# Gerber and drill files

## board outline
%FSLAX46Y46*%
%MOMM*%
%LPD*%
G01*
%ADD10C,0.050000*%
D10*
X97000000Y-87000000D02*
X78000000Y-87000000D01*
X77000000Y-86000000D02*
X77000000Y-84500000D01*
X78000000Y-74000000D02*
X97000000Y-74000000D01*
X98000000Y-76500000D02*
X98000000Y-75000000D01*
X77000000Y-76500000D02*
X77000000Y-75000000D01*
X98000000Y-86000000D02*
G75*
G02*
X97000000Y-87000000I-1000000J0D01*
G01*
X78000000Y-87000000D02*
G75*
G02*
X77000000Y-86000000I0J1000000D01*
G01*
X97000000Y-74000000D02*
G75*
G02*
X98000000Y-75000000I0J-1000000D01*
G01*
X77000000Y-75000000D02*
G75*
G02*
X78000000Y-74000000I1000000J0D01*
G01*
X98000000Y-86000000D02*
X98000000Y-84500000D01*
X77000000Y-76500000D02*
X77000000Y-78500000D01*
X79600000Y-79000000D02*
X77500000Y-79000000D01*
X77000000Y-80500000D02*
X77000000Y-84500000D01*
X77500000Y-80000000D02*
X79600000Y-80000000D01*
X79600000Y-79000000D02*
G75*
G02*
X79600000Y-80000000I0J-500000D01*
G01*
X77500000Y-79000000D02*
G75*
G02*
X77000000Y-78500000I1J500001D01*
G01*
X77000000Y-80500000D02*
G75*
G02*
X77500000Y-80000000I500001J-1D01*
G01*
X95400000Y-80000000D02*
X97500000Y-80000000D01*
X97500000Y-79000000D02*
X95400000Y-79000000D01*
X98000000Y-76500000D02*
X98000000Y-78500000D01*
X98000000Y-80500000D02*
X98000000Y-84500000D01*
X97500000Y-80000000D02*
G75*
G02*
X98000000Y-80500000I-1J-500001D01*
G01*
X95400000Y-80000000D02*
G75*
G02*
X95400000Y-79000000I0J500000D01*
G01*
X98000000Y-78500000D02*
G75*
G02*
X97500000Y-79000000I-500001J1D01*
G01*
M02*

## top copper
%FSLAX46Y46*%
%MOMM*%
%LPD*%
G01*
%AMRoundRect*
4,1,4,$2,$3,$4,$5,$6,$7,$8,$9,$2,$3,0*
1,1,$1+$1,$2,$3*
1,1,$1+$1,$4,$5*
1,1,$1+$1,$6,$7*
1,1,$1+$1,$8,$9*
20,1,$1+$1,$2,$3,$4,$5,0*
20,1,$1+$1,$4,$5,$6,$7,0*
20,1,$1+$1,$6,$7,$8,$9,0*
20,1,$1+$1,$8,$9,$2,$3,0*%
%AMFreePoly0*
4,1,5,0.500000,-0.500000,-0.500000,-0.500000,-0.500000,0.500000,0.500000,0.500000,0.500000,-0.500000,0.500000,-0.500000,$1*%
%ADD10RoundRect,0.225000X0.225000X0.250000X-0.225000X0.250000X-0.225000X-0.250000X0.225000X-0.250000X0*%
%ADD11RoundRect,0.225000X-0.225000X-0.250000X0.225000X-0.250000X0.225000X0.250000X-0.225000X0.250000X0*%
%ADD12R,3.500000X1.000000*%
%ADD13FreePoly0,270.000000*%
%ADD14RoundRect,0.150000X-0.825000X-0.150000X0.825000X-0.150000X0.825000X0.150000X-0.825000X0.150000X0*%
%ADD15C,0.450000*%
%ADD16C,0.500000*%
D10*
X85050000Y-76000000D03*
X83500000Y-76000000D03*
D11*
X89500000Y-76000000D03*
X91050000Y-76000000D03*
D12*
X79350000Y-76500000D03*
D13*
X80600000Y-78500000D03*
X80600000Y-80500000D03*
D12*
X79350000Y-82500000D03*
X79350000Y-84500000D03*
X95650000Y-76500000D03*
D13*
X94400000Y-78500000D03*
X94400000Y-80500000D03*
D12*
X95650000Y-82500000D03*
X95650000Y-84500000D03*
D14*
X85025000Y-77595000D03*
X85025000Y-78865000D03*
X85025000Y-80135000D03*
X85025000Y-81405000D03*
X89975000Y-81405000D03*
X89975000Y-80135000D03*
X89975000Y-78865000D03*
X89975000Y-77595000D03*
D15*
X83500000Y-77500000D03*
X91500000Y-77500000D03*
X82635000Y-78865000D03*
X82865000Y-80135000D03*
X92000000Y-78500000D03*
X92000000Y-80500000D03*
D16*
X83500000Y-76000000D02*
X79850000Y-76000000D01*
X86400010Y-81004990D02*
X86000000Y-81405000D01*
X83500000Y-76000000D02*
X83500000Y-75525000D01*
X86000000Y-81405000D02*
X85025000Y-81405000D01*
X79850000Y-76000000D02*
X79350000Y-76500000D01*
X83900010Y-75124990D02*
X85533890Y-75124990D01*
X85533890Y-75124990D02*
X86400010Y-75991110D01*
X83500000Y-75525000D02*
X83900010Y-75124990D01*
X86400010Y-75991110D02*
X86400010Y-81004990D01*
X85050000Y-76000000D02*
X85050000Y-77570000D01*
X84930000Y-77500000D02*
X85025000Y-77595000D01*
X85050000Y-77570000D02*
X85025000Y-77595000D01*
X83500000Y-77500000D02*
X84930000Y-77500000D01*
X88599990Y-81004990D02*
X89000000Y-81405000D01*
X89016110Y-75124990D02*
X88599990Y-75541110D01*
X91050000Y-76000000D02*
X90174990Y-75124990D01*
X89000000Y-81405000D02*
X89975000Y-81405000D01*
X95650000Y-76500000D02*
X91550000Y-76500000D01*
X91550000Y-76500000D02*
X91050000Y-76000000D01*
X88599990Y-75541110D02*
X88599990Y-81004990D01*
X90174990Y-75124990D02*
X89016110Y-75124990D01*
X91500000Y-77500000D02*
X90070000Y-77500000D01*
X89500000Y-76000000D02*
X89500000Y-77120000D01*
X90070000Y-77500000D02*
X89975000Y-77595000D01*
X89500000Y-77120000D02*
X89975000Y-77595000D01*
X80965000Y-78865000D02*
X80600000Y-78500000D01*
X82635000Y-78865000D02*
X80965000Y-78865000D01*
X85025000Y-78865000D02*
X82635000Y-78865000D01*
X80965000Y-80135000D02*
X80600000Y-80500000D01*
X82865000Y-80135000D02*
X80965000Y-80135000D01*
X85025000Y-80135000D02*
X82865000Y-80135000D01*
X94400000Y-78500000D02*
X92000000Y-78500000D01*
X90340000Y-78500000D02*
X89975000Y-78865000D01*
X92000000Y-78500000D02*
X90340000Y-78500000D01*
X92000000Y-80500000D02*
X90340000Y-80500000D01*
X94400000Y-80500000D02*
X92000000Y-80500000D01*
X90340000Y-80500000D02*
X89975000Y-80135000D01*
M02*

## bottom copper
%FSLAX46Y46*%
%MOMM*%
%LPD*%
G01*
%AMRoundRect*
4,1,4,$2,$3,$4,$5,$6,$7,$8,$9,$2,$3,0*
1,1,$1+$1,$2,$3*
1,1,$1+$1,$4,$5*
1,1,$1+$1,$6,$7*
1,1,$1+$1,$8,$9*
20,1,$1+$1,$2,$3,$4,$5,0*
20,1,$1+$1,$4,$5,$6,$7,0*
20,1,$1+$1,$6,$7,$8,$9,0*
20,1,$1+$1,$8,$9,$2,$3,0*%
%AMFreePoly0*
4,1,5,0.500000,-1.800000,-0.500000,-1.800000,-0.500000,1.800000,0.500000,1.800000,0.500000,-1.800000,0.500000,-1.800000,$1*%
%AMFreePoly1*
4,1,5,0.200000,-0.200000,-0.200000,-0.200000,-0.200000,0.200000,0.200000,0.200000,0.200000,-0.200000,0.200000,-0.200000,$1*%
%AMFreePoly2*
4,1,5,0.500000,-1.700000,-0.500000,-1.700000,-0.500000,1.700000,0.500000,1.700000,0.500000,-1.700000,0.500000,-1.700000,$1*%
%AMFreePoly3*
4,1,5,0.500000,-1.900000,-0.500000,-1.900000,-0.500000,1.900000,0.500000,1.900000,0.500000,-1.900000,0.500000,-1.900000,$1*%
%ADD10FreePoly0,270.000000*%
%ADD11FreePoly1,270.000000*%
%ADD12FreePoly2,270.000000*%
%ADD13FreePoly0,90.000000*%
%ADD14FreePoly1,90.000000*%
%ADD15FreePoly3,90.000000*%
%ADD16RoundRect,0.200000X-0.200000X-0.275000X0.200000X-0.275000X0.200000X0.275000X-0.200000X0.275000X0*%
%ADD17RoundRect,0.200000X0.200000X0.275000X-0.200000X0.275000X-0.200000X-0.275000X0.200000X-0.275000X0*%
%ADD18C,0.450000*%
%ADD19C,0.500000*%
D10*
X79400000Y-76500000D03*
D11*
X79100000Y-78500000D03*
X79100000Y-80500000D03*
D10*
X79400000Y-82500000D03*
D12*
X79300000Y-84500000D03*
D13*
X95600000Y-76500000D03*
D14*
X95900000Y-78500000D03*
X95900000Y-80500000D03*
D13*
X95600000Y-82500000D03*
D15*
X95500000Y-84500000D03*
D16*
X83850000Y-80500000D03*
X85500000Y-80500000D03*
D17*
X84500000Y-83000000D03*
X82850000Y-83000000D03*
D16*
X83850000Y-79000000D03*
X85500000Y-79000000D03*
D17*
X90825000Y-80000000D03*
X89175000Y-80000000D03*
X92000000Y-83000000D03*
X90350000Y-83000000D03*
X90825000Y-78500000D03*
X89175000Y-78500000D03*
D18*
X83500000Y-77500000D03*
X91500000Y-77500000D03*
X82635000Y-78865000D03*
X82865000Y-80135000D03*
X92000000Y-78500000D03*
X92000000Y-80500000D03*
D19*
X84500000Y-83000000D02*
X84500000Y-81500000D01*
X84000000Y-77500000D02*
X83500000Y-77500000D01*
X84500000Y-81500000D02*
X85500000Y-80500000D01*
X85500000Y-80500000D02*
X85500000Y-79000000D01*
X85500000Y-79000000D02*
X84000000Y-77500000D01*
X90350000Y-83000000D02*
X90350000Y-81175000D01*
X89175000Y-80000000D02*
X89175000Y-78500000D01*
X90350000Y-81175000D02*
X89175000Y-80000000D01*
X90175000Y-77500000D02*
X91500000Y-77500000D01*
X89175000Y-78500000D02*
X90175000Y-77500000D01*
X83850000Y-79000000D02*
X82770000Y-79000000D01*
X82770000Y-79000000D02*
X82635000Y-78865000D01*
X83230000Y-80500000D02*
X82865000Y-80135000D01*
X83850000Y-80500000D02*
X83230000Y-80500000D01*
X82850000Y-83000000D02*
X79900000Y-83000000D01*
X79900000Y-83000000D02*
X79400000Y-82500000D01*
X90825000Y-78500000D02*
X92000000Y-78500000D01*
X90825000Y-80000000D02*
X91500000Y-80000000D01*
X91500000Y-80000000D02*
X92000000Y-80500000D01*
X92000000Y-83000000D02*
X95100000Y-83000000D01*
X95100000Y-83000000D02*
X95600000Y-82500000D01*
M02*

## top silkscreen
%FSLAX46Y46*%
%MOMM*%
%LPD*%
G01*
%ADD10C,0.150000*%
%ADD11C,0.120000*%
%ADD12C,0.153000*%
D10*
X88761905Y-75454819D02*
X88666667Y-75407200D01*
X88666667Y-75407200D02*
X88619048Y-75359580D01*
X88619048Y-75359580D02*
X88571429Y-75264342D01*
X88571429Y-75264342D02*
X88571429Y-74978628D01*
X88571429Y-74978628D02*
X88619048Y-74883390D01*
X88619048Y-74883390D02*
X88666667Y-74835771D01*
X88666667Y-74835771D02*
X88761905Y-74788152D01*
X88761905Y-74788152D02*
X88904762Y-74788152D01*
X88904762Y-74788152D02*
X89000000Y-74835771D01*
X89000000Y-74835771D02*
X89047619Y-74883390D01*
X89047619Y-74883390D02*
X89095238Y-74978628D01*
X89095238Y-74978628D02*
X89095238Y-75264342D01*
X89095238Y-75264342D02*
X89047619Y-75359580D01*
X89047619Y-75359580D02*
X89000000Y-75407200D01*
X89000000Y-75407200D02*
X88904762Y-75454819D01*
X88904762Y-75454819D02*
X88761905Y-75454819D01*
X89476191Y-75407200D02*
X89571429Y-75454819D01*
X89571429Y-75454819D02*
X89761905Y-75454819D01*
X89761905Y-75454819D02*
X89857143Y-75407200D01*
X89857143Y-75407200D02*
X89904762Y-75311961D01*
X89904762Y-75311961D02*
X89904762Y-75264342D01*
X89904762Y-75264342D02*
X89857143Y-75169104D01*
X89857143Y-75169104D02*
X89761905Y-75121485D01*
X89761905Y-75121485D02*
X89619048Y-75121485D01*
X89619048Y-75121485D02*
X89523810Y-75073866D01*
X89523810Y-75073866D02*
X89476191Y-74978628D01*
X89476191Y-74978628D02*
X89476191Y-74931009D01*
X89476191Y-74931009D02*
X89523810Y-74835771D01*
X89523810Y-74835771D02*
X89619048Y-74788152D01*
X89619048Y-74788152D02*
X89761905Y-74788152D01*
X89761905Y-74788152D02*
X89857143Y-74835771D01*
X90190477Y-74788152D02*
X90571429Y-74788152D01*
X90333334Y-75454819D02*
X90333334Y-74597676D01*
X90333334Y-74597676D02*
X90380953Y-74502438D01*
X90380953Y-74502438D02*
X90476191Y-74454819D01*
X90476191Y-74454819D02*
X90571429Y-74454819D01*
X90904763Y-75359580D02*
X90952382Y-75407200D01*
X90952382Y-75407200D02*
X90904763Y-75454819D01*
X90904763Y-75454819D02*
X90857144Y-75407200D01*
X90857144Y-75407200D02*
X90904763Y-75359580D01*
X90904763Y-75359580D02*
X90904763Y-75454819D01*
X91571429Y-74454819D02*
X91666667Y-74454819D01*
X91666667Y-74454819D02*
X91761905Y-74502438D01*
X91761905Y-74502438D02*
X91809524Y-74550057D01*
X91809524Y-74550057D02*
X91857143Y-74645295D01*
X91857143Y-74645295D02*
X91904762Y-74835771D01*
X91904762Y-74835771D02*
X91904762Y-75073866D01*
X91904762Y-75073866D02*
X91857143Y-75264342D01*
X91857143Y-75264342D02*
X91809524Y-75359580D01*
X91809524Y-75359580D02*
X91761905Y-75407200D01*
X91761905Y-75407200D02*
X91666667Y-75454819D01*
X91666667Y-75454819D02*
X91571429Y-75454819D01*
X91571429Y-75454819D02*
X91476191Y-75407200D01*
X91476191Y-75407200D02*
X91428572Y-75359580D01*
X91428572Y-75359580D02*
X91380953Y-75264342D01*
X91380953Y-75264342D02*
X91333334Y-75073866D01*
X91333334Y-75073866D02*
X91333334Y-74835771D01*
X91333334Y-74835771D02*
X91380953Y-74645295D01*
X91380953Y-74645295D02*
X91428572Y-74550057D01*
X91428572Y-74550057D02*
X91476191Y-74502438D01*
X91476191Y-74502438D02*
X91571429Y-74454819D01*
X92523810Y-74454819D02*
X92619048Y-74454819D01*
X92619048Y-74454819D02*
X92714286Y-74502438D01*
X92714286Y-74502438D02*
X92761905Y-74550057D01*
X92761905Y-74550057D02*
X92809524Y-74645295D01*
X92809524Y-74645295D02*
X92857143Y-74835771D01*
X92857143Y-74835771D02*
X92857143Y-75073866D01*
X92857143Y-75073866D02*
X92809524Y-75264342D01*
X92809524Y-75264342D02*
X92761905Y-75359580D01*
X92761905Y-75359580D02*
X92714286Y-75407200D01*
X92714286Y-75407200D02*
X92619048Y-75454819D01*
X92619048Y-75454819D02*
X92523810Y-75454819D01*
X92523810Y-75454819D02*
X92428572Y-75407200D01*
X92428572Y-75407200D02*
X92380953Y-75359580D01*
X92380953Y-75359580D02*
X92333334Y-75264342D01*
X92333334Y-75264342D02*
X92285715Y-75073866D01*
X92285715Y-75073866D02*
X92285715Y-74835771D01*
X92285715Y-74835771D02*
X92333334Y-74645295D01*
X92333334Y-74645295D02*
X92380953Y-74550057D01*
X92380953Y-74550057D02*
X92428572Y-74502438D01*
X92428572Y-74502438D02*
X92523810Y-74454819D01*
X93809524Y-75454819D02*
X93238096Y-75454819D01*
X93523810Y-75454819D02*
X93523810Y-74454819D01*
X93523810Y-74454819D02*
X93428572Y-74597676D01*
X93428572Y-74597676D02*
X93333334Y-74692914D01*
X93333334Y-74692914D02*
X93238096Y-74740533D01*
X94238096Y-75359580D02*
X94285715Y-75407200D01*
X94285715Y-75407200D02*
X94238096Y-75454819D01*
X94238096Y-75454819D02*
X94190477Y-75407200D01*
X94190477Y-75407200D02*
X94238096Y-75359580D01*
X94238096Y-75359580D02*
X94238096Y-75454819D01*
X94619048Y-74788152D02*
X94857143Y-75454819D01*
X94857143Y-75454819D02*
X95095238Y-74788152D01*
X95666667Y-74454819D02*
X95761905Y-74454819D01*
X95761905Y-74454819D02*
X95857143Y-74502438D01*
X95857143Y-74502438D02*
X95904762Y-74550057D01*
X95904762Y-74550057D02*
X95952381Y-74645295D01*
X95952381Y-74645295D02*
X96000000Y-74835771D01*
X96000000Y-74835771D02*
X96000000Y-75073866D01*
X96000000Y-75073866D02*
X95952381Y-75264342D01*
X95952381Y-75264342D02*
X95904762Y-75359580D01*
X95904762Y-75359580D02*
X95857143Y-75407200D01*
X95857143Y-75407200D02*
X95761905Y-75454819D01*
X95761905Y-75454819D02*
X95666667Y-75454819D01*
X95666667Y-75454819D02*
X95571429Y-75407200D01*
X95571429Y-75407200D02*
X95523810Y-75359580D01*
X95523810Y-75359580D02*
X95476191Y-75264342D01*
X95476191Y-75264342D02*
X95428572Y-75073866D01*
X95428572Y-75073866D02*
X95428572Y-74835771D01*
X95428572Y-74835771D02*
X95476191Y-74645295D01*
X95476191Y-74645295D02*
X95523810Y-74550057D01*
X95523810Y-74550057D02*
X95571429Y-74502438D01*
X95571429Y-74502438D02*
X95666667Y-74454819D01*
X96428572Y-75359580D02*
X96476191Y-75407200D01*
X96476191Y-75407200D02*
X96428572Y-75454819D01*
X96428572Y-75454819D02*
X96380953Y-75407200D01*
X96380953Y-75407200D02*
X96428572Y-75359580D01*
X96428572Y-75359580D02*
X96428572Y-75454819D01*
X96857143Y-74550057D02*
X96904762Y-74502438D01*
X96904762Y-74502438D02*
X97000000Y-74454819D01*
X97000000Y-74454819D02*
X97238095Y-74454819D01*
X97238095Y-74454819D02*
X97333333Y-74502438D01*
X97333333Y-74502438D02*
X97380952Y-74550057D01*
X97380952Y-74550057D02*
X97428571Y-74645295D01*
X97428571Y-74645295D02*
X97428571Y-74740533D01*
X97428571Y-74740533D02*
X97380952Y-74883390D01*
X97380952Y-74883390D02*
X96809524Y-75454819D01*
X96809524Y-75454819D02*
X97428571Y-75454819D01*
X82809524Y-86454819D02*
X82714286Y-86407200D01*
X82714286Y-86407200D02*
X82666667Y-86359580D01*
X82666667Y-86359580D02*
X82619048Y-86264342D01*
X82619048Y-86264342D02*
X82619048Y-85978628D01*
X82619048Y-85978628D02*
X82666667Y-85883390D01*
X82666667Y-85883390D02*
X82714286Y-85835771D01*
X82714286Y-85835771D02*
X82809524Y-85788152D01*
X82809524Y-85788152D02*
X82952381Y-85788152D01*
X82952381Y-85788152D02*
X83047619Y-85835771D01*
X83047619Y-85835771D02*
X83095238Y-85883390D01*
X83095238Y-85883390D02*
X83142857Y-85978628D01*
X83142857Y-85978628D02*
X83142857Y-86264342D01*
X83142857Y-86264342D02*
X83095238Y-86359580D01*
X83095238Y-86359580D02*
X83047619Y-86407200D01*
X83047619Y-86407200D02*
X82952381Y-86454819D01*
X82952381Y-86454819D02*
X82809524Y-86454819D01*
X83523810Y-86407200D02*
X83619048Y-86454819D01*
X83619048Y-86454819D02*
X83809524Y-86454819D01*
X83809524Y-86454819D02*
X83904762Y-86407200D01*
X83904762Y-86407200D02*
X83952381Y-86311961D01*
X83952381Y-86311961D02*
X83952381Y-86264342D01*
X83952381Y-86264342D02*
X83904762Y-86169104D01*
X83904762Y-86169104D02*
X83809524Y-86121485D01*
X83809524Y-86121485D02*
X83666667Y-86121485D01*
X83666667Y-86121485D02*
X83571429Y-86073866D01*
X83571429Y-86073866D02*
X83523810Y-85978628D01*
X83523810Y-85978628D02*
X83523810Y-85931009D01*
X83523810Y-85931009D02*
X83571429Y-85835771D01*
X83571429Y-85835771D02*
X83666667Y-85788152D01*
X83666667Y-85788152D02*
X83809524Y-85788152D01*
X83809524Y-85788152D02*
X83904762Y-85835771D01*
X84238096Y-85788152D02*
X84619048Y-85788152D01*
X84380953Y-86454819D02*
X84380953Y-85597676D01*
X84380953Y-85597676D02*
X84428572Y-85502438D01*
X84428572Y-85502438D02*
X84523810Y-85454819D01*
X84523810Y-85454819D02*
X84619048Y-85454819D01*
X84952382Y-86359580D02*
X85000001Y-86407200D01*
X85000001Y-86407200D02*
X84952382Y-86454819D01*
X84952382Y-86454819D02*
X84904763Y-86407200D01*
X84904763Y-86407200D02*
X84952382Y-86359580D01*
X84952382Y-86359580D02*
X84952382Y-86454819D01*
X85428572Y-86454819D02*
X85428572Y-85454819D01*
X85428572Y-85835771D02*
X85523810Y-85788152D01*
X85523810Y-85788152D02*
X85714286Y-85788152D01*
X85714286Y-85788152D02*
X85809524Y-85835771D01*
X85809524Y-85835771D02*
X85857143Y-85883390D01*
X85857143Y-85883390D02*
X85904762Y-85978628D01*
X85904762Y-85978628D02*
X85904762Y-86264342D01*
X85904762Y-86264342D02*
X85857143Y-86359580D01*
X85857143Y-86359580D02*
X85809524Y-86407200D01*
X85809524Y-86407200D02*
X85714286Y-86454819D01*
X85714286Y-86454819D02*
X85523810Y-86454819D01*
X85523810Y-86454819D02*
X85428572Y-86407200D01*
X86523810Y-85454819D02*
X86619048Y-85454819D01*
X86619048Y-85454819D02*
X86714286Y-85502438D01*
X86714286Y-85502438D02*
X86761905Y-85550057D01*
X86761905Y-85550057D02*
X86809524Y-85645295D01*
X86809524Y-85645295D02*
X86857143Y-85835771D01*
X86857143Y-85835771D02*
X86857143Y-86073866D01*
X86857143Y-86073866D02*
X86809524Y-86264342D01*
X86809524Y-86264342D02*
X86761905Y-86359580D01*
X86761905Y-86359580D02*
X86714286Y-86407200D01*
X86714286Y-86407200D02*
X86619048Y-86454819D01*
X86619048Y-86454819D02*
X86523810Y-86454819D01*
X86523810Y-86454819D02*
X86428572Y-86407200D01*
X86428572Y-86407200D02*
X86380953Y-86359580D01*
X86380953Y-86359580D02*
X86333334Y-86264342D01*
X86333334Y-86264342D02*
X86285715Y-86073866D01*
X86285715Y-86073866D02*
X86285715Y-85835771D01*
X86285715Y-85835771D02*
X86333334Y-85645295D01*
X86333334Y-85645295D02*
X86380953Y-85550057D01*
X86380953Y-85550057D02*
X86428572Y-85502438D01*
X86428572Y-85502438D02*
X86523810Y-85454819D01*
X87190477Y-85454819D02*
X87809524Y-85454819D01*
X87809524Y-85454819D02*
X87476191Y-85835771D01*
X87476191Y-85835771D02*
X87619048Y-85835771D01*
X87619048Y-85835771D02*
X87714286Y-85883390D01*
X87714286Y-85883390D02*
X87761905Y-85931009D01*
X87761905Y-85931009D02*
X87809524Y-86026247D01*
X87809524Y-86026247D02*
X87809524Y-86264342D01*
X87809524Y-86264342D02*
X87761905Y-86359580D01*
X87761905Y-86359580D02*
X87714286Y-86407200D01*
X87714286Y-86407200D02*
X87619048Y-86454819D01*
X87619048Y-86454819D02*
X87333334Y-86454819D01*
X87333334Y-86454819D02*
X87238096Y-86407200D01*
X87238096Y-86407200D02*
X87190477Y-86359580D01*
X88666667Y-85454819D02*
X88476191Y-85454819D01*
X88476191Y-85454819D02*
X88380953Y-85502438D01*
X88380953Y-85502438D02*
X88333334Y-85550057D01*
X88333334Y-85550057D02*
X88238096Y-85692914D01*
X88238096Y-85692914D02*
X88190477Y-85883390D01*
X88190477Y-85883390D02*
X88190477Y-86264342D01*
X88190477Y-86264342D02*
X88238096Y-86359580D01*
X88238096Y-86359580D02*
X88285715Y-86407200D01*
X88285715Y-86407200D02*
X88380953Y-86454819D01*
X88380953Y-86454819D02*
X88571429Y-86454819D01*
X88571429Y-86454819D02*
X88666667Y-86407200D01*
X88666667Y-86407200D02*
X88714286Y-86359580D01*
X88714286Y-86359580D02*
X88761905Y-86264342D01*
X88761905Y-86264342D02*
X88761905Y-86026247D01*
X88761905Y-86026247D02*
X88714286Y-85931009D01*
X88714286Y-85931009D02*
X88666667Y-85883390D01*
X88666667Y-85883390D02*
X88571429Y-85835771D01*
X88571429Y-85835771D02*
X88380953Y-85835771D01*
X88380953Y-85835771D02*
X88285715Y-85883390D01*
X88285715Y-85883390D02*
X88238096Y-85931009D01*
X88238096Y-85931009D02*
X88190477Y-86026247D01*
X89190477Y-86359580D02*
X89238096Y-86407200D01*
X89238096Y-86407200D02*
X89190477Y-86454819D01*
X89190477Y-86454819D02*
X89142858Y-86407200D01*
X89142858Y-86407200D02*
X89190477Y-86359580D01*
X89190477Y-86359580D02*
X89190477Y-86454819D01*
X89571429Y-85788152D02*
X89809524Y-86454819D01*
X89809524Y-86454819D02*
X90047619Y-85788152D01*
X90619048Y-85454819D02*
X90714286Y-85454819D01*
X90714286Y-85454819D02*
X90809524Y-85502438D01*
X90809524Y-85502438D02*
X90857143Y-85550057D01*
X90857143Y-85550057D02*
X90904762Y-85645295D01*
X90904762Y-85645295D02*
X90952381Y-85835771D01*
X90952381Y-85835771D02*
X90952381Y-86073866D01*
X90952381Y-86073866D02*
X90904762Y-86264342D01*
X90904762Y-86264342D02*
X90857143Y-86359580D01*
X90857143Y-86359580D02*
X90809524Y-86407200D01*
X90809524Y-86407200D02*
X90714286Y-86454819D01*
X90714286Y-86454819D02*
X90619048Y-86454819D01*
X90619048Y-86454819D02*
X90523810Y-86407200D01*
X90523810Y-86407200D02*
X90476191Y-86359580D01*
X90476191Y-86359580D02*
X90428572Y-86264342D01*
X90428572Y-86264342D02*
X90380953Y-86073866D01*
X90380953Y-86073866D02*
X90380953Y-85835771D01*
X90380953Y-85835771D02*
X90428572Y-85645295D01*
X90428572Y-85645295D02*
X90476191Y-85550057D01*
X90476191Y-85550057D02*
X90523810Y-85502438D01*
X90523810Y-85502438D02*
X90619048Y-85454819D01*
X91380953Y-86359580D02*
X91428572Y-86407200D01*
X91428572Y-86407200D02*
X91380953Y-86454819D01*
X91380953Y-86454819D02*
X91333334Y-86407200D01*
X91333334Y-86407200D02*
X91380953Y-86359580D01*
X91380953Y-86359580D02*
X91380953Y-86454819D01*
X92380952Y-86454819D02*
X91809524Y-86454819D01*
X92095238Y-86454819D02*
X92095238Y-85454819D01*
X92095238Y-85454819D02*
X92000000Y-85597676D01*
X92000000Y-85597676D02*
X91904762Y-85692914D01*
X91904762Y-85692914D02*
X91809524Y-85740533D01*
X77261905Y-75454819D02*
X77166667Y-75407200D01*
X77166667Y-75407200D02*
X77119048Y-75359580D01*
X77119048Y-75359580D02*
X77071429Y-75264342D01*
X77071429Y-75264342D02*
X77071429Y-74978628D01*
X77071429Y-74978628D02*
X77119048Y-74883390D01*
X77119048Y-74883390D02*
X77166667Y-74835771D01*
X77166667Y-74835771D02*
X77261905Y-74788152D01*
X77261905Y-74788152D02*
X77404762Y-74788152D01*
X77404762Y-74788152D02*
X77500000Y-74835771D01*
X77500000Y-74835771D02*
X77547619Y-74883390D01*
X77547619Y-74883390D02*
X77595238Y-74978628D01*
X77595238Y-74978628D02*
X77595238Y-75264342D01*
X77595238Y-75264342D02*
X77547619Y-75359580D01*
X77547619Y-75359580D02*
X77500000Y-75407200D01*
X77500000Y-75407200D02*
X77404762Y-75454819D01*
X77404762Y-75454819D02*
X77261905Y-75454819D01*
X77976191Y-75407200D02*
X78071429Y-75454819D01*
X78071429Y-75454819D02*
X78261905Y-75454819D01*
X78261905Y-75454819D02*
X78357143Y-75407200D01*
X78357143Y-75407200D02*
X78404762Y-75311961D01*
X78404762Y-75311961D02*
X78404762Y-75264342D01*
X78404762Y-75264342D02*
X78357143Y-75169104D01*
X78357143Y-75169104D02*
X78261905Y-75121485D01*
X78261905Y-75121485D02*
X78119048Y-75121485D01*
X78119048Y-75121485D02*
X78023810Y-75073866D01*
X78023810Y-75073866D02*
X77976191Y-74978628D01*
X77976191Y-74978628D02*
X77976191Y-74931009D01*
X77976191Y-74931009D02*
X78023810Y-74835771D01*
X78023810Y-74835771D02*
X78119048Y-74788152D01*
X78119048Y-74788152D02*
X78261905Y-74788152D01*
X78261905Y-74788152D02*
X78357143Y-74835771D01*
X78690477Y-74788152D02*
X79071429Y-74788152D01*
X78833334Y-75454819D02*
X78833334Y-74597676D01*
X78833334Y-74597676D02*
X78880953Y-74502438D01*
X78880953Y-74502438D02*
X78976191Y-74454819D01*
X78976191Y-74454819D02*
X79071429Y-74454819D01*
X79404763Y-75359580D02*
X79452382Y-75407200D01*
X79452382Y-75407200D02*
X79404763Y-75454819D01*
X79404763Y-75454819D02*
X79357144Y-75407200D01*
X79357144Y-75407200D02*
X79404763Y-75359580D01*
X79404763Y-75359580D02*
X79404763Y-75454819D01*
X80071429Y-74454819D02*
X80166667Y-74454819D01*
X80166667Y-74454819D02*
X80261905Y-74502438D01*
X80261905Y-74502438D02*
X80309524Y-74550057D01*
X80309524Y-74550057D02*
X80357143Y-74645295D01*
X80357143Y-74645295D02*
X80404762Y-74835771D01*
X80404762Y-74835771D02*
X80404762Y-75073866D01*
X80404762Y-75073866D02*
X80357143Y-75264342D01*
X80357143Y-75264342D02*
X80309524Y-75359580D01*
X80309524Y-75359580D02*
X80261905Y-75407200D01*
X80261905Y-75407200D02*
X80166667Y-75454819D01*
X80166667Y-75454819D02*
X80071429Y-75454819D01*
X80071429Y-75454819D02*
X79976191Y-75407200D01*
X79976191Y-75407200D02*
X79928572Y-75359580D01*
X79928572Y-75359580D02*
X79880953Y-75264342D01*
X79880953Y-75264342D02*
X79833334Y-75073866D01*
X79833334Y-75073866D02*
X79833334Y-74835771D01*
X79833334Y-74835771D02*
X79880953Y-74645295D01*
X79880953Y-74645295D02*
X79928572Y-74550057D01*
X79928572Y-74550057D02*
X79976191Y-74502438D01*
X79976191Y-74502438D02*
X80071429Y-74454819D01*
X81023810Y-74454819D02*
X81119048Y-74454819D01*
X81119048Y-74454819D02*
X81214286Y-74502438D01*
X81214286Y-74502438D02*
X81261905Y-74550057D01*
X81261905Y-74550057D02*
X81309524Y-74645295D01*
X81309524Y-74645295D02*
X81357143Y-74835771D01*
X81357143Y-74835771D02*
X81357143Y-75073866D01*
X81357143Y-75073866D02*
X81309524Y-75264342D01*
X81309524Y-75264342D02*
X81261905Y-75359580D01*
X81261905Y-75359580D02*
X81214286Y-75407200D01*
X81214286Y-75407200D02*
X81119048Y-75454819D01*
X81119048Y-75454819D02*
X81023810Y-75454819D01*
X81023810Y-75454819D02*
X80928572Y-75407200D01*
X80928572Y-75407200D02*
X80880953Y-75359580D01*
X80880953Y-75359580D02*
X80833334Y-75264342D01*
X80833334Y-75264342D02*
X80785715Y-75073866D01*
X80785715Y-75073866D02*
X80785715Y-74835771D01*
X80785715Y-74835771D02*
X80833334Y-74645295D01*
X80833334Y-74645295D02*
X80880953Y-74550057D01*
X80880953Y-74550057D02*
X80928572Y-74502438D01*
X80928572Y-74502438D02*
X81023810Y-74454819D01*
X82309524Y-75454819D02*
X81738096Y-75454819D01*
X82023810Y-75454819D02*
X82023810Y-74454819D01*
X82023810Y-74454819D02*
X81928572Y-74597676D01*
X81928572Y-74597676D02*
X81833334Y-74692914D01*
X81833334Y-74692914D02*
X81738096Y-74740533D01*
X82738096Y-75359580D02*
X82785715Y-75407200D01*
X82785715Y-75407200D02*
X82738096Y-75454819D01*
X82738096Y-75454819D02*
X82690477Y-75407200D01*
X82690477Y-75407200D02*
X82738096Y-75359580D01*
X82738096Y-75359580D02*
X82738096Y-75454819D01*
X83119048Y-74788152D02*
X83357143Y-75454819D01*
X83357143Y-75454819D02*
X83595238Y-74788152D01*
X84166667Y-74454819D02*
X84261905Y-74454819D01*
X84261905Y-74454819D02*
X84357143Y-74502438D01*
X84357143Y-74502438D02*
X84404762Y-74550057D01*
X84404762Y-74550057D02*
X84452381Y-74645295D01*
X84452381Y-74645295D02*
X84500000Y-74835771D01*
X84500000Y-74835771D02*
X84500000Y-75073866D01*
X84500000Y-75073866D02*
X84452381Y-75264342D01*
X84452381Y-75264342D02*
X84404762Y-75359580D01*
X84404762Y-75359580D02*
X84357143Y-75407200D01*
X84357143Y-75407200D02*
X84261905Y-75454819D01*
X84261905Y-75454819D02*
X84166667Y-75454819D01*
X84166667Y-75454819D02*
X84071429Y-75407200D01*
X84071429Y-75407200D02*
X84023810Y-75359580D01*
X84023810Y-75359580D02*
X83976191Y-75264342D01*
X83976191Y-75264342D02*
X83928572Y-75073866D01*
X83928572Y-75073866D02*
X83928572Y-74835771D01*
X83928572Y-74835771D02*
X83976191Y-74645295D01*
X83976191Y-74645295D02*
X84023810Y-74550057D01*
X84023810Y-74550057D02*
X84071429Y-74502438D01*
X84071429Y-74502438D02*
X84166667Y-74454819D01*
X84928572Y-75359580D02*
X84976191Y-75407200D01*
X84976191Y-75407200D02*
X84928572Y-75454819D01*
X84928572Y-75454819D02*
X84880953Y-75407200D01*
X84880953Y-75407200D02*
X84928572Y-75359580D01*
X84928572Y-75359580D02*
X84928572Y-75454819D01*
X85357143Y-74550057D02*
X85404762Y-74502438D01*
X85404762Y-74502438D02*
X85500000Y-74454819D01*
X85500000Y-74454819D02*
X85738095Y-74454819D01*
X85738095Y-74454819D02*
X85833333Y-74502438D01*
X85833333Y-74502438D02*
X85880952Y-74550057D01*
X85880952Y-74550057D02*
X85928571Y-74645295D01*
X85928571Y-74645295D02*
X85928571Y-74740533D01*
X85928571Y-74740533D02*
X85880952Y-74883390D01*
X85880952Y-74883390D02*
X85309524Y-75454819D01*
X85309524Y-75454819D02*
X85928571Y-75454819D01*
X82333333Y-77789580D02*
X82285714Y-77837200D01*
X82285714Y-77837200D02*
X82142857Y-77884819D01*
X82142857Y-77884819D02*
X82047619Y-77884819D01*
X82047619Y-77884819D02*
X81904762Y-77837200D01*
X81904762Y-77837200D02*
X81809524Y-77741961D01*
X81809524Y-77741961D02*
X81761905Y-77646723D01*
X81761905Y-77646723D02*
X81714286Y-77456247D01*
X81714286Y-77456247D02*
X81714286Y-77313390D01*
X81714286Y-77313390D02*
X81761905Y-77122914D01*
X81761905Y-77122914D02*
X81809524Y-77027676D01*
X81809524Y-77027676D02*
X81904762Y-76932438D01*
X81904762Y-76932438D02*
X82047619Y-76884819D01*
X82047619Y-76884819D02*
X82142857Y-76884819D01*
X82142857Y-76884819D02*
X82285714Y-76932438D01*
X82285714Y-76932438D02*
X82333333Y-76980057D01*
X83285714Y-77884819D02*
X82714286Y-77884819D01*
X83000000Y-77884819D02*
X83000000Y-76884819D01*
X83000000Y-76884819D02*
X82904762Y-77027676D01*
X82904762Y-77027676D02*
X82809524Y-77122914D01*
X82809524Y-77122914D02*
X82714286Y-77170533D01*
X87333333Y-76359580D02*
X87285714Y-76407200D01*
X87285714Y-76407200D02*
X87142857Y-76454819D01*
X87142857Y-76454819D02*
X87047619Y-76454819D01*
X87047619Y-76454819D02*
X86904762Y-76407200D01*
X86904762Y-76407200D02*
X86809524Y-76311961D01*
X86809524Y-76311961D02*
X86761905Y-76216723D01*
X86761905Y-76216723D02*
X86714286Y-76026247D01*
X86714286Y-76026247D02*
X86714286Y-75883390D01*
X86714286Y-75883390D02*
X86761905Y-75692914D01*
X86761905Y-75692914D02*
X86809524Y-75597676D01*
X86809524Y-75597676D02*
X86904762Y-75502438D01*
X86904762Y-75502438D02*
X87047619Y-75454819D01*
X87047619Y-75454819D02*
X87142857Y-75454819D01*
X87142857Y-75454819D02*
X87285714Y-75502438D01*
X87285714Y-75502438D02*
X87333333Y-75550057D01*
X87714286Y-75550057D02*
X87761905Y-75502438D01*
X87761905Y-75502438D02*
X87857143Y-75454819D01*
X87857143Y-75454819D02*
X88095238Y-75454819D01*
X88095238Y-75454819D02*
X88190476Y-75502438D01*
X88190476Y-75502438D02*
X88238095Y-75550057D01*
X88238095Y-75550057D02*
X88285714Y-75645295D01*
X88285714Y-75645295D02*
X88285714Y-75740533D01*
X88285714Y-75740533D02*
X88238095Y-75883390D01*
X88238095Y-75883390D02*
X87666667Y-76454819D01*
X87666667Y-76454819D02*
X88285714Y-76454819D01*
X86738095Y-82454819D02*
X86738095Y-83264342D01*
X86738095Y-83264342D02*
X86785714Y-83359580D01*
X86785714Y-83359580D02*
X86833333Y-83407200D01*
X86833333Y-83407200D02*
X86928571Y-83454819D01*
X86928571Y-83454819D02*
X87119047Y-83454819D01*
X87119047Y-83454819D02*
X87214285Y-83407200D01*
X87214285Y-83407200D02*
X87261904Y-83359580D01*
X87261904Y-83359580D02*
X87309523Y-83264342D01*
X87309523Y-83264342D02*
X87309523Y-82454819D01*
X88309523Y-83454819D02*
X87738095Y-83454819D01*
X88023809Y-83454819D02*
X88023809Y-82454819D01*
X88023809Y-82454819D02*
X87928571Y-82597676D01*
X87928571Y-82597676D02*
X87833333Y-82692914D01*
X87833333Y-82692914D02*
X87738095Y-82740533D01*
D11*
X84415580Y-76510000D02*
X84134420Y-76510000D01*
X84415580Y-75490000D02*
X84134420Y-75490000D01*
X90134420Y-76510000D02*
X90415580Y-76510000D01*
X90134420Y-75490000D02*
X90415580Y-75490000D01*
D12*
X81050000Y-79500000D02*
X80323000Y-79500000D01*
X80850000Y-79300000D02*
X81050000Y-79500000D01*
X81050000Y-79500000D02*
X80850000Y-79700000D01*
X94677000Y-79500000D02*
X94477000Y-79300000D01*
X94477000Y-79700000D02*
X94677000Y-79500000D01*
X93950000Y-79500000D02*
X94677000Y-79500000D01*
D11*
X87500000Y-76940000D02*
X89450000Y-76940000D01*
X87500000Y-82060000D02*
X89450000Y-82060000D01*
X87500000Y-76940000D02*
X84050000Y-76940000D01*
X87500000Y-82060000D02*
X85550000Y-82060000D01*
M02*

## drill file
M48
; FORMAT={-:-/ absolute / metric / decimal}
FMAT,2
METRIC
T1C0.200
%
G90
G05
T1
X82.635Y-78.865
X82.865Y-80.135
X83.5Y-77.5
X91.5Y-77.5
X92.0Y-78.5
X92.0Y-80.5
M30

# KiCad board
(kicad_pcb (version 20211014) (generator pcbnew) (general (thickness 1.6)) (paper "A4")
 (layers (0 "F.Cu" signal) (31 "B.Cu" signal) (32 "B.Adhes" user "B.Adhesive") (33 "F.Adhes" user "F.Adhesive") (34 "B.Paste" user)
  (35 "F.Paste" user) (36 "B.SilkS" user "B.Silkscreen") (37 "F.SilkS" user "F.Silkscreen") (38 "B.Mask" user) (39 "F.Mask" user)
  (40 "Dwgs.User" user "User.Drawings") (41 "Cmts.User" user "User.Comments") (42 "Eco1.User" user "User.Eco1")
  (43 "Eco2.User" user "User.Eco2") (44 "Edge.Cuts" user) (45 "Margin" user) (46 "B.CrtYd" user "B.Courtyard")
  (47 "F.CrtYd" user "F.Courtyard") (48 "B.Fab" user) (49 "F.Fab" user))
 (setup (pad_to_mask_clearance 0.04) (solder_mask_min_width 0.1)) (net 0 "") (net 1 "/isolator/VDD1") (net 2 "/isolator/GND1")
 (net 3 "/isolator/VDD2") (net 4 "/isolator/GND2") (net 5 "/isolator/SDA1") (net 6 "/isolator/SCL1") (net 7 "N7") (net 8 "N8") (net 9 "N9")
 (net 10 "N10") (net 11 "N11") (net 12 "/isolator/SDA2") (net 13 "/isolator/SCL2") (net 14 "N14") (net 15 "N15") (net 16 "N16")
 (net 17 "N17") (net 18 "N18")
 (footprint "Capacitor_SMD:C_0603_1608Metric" (layer "F.Cu") (at 84.275 76 180)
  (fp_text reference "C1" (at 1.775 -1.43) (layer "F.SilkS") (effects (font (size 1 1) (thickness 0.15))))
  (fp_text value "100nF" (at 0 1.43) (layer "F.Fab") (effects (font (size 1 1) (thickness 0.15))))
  (fp_line (start -0.14058 -0.51) (end 0.14058 -0.51) (layer "F.SilkS") (width 0.12))
  (fp_line (start -0.14058 0.51) (end 0.14058 0.51) (layer "F.SilkS") (width 0.12))
  (pad "1" smd roundrect locked (at -0.775 0 180) (size 0.9 0.95) (layers "F.Cu" "F.Paste" "F.Mask") (roundrect_rratio 0.25)
   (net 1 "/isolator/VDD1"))
  (pad "2" smd roundrect locked (at 0.775 0 180) (size 0.9 0.95) (layers "F.Cu" "F.Paste" "F.Mask") (roundrect_rratio 0.25)
   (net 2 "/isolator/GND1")))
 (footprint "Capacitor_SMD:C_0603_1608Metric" (layer "F.Cu") (at 90.275 76)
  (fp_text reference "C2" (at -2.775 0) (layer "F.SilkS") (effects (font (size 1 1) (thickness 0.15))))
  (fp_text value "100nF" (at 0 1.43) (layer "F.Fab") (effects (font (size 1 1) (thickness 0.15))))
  (fp_line (start -0.14058 0.51) (end 0.14058 0.51) (layer "F.SilkS") (width 0.12))
  (fp_line (start -0.14058 -0.51) (end 0.14058 -0.51) (layer "F.SilkS") (width 0.12))
  (pad "1" smd roundrect locked (at -0.775 0) (size 0.9 0.95) (layers "F.Cu" "F.Paste" "F.Mask") (roundrect_rratio 0.25)
   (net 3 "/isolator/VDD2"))
  (pad "2" smd roundrect locked (at 0.775 0) (size 0.9 0.95) (layers "F.Cu" "F.Paste" "F.Mask") (roundrect_rratio 0.25)
   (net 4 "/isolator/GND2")))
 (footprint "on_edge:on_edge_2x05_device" (layer "F.Cu") (at 77 80.5 -90)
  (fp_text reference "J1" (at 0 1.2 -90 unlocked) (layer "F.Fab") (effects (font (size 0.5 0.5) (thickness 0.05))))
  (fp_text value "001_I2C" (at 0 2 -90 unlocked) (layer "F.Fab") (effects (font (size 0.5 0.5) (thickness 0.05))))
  (fp_line (start -1 -4.05) (end -1 -3.323) (layer "F.SilkS") (width 0.153))
  (fp_line (start -1.2 -3.85) (end -1 -4.05) (layer "F.SilkS") (width 0.153))
  (fp_line (start -1 -4.05) (end -0.8 -3.85) (layer "F.SilkS") (width 0.153))
  (fp_line (start -4 0) (end -2 0) (layer "Edge.Cuts") (width 0.05))
  (fp_line (start -1.5 -2.6) (end -1.5 -0.5) (layer "Edge.Cuts") (width 0.05))
  (fp_line (start 0 0) (end 4 0) (layer "Edge.Cuts") (width 0.05))
  (fp_line (start -0.5 -0.5) (end -0.5 -2.6) (layer "Edge.Cuts") (width 0.05))
  (fp_arc (start -1.5 -2.6) (mid -1 -3.1) (end -0.5 -2.6) (layer "Edge.Cuts") (width 0.05))
  (fp_arc (start -1.5 -0.5) (mid -1.646447 -0.146447) (end -2 0) (layer "Edge.Cuts") (width 0.05))
  (fp_arc (start 0 0) (mid -0.353553 -0.146447) (end -0.5 -0.5) (layer "Edge.Cuts") (width 0.05))
  (pad "1" smd rect locked (at -4 -2.35 90) (size 1 3.5) (layers "F.Cu" "F.Mask") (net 2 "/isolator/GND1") (zone_connect 0))
  (pad "2" smd custom locked (at -2 -3.6 270) (size 1 1) (layers "F.Cu" "F.Mask") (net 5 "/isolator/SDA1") (zone_connect 0)
   (options (clearance outline) (anchor rect)) (primitives))
  (pad "3" smd custom locked (at 0 -3.6 270) (size 1 1) (layers "F.Cu" "F.Mask") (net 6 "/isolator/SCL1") (zone_connect 0)
   (options (clearance outline) (anchor rect)) (primitives))
  (pad "4" smd rect locked (at 2 -2.35 90) (size 1 3.5) (layers "F.Cu" "F.Mask") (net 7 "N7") (zone_connect 0))
  (pad "5" smd rect locked (at 4 -2.35 90) (size 1 3.5) (layers "F.Cu" "F.Mask") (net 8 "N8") (zone_connect 0))
  (pad "6" smd custom locked (at -4 -2.4 270) (size 1 3.6) (layers "B.Cu" "B.Mask") (zone_connect 0)
   (options (clearance outline) (anchor rect)) (primitives))
  (pad "7" smd custom locked (at -2 -2.1 270) (size 0.4 0.4) (layers "B.Cu" "B.Mask") (zone_connect 0)
   (options (clearance outline) (anchor rect)) (primitives))
  (pad "8" smd custom locked (at 0 -2.1 270) (size 0.4 0.4) (layers "B.Cu" "B.Mask") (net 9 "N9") (zone_connect 0)
   (options (clearance outline) (anchor rect)) (primitives))
  (pad "9" smd custom locked (at 2 -2.4 270) (size 1 3.6) (layers "B.Cu" "B.Mask") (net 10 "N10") (zone_connect 0)
   (options (clearance outline) (anchor rect)) (primitives))
  (pad "10" smd custom locked (at 4 -2.3 270) (size 1 3.4) (layers "B.Cu" "B.Mask") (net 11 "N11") (zone_connect 0)
   (options (clearance outline) (anchor rect)) (primitives)))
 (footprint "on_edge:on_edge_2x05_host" (layer "F.Cu") (at 98 80.5 -90)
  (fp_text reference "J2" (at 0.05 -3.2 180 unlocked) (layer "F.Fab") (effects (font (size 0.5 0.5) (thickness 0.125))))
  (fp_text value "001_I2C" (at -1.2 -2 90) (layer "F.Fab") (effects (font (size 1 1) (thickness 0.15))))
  (fp_line (start -1 3.323) (end -1.2 3.523) (layer "F.SilkS") (width 0.153))
  (fp_line (start -0.8 3.523) (end -1 3.323) (layer "F.SilkS") (width 0.153))
  (fp_line (start -1 4.05) (end -1 3.323) (layer "F.SilkS") (width 0.153))
  (fp_line (start -0.5 2.6) (end -0.5 0.5) (layer "Edge.Cuts") (width 0.05))
  (fp_line (start -1.5 0.5) (end -1.5 2.6) (layer "Edge.Cuts") (width 0.05))
  (fp_line (start -4 0) (end -2 0) (layer "Edge.Cuts") (width 0.05))
  (fp_line (start 0 0) (end 4 0) (layer "Edge.Cuts") (width 0.05))
  (fp_arc (start -0.5 0.5) (mid -0.353553 0.146447) (end 0 0) (layer "Edge.Cuts") (width 0.05))
  (fp_arc (start -0.5 2.6) (mid -1 3.1) (end -1.5 2.6) (layer "Edge.Cuts") (width 0.05))
  (fp_arc (start -2 0) (mid -1.646447 0.146447) (end -1.5 0.5) (layer "Edge.Cuts") (width 0.05))
  (pad "1" smd rect locked (at -4 2.35 270) (size 1 3.5) (layers "F.Cu" "F.Mask") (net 4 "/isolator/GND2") (zone_connect 0))
  (pad "2" smd custom locked (at -2 3.6 270) (size 1 1) (layers "F.Cu" "F.Mask") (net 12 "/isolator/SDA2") (zone_connect 0)
   (options (clearance outline) (anchor rect)) (primitives))
  (pad "3" smd custom locked (at 0 3.6 270) (size 1 1) (layers "F.Cu" "F.Mask") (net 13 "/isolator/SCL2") (zone_connect 0)
   (options (clearance outline) (anchor rect)) (primitives))
  (pad "4" smd rect locked (at 2 2.35 270) (size 1 3.5) (layers "F.Cu" "F.Mask") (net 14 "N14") (zone_connect 0))
  (pad "5" smd rect locked (at 4 2.35 270) (size 1 3.5) (layers "F.Cu" "F.Mask") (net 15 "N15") (zone_connect 0))
  (pad "6" smd custom locked (at -4 2.4 90) (size 1 3.6) (layers "B.Cu" "B.Mask") (zone_connect 0)
   (options (clearance outline) (anchor rect)) (primitives))
  (pad "7" smd custom locked (at -2 2.1 90) (size 0.4 0.4) (layers "B.Cu" "B.Mask") (zone_connect 0)
   (options (clearance outline) (anchor rect)) (primitives))
  (pad "8" smd custom locked (at 0 2.1 90) (size 0.4 0.4) (layers "B.Cu" "B.Mask") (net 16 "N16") (zone_connect 0)
   (options (clearance outline) (anchor rect)) (primitives))
  (pad "9" smd custom locked (at 2 2.4 90) (size 1 3.6) (layers "B.Cu" "B.Mask") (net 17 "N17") (zone_connect 0)
   (options (clearance outline) (anchor rect)) (primitives))
  (pad "10" smd custom locked (at 4 2.5 90) (size 1 3.8) (layers "B.Cu" "B.Mask") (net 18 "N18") (zone_connect 0)
   (options (clearance outline) (anchor rect)) (primitives)))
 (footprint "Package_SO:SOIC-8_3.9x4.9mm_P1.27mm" (layer "F.Cu") (at 87.5 79.5)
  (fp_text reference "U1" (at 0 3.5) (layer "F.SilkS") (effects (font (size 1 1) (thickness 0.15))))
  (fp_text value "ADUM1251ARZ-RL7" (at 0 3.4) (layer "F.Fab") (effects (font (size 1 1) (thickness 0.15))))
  (fp_line (start 0 -2.56) (end 1.95 -2.56) (layer "F.SilkS") (width 0.12))
  (fp_line (start 0 2.56) (end 1.95 2.56) (layer "F.SilkS") (width 0.12))
  (fp_line (start 0 -2.56) (end -3.45 -2.56) (layer "F.SilkS") (width 0.12))
  (fp_line (start 0 2.56) (end -1.95 2.56) (layer "F.SilkS") (width 0.12))
  (pad "1" smd roundrect locked (at -2.475 -1.905) (size 1.95 0.6) (layers "F.Cu" "F.Paste" "F.Mask") (roundrect_rratio 0.25)
   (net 1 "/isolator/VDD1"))
  (pad "2" smd roundrect locked (at -2.475 -0.635) (size 1.95 0.6) (layers "F.Cu" "F.Paste" "F.Mask") (roundrect_rratio 0.25)
   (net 5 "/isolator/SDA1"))
  (pad "3" smd roundrect locked (at -2.475 0.635) (size 1.95 0.6) (layers "F.Cu" "F.Paste" "F.Mask") (roundrect_rratio 0.25)
   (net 6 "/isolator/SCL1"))
  (pad "4" smd roundrect locked (at -2.475 1.905) (size 1.95 0.6) (layers "F.Cu" "F.Paste" "F.Mask") (roundrect_rratio 0.25)
   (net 2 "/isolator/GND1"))
  (pad "5" smd roundrect locked (at 2.475 1.905) (size 1.95 0.6) (layers "F.Cu" "F.Paste" "F.Mask") (roundrect_rratio 0.25)
   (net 4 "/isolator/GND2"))
  (pad "6" smd roundrect locked (at 2.475 0.635) (size 1.95 0.6) (layers "F.Cu" "F.Paste" "F.Mask") (roundrect_rratio 0.25)
   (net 13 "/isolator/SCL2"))
  (pad "7" smd roundrect locked (at 2.475 -0.635) (size 1.95 0.6) (layers "F.Cu" "F.Paste" "F.Mask") (roundrect_rratio 0.25)
   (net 12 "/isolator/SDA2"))
  (pad "8" smd roundrect locked (at 2.475 -1.905) (size 1.95 0.6) (layers "F.Cu" "F.Paste" "F.Mask") (roundrect_rratio 0.25)
   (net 3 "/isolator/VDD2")))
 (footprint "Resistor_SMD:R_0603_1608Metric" (layer "B.Cu") (at 84.675 80.5)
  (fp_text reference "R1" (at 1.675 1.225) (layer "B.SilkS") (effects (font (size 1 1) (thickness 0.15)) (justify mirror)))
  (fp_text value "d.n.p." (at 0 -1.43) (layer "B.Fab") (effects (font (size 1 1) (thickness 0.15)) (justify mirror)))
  (pad "1" smd roundrect locked (at -0.825 0) (size 0.8 0.95) (layers "B.Cu" "B.Paste" "B.Mask") (roundrect_rratio 0.25)
   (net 6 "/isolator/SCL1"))
  (pad "2" smd roundrect locked (at 0.825 0) (size 0.8 0.95) (layers "B.Cu" "B.Paste" "B.Mask") (roundrect_rratio 0.25)
   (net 1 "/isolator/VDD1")))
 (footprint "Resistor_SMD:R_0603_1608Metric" (layer "B.Cu") (at 83.675 83 180)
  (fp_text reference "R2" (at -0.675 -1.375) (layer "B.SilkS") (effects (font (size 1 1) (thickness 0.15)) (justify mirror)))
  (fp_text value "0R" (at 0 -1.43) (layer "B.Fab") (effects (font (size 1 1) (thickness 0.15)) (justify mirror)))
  (pad "1" smd roundrect locked (at -0.825 0 180) (size 0.8 0.95) (layers "B.Cu" "B.Paste" "B.Mask") (roundrect_rratio 0.25)
   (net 1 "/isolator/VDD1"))
  (pad "2" smd roundrect locked (at 0.825 0 180) (size 0.8 0.95) (layers "B.Cu" "B.Paste" "B.Mask") (roundrect_rratio 0.25) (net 10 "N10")))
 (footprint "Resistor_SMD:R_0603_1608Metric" (layer "B.Cu") (at 84.675 79)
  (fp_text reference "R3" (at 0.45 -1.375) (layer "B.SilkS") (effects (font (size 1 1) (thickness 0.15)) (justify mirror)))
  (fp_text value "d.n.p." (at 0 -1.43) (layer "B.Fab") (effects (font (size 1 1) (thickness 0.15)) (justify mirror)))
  (pad "1" smd roundrect locked (at -0.825 0) (size 0.8 0.95) (layers "B.Cu" "B.Paste" "B.Mask") (roundrect_rratio 0.25)
   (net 5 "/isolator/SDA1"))
  (pad "2" smd roundrect locked (at 0.825 0) (size 0.8 0.95) (layers "B.Cu" "B.Paste" "B.Mask") (roundrect_rratio 0.25)
   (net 1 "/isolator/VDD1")))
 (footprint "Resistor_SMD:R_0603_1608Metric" (layer "B.Cu") (at 90 80 180)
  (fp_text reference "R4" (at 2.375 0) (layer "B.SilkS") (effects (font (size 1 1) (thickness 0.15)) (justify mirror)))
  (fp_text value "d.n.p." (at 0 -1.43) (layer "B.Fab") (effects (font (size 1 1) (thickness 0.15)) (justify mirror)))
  (pad "1" smd roundrect locked (at -0.825 0 180) (size 0.8 0.95) (layers "B.Cu" "B.Paste" "B.Mask") (roundrect_rratio 0.25)
   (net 13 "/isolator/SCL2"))
  (pad "2" smd roundrect locked (at 0.825 0 180) (size 0.8 0.95) (layers "B.Cu" "B.Paste" "B.Mask") (roundrect_rratio 0.25)
   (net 3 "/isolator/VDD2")))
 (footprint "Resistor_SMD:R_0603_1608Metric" (layer "B.Cu") (at 91.175 83 180)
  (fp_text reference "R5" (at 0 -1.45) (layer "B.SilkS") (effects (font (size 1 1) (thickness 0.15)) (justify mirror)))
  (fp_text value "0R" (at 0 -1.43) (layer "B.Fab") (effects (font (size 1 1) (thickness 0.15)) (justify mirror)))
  (pad "1" smd roundrect locked (at -0.825 0 180) (size 0.8 0.95) (layers "B.Cu" "B.Paste" "B.Mask") (roundrect_rratio 0.25) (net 17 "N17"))
  (pad "2" smd roundrect locked (at 0.825 0 180) (size 0.8 0.95) (layers "B.Cu" "B.Paste" "B.Mask") (roundrect_rratio 0.25)
   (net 3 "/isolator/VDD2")))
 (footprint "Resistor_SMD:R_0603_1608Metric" (layer "B.Cu") (at 90 78.5 180)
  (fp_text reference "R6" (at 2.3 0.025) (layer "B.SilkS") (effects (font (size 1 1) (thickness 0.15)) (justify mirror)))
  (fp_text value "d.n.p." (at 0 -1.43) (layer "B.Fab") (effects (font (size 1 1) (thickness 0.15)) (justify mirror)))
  (pad "1" smd roundrect locked (at -0.825 0 180) (size 0.8 0.95) (layers "B.Cu" "B.Paste" "B.Mask") (roundrect_rratio 0.25)
   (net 12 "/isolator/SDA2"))
  (pad "2" smd roundrect locked (at 0.825 0 180) (size 0.8 0.95) (layers "B.Cu" "B.Paste" "B.Mask") (roundrect_rratio 0.25)
   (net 3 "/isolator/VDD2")))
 (gr_line (start 97 87) (end 78 87) (layer "Edge.Cuts") (width 0.05))
 (gr_line (start 77 86) (end 77 84.5) (layer "Edge.Cuts") (width 0.05))
 (gr_line (start 78 74) (end 97 74) (layer "Edge.Cuts") (width 0.05))
 (gr_line (start 98 76.5) (end 98 75) (layer "Edge.Cuts") (width 0.05))
 (gr_line (start 77 76.5) (end 77 75) (layer "Edge.Cuts") (width 0.05))
 (gr_arc (start 98 86) (mid 97.707107 86.707107) (end 97 87) (layer "Edge.Cuts") (width 0.05))
 (gr_arc (start 78 87) (mid 77.292893 86.707107) (end 77 86) (layer "Edge.Cuts") (width 0.05))
 (gr_arc (start 97 74) (mid 97.707107 74.292893) (end 98 75) (layer "Edge.Cuts") (width 0.05))
 (gr_arc (start 77 75) (mid 77.292893 74.292893) (end 78 74) (layer "Edge.Cuts") (width 0.05))
 (gr_line (start 98 86) (end 98 84.5) (layer "Edge.Cuts") (width 0.05))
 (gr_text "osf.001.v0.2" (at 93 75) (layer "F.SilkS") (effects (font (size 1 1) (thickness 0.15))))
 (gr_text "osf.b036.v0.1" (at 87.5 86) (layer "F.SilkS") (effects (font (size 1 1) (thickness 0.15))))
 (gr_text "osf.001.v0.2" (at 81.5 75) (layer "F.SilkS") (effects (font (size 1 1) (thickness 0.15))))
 (segment (start 83.5 76) (end 79.85 76) (width 0.5) (layer "F.Cu") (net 2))
 (segment (start 86.40001 81.00499) (end 86 81.405) (width 0.5) (layer "F.Cu") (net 2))
 (segment (start 83.5 76) (end 83.5 75.525) (width 0.5) (layer "F.Cu") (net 2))
 (segment (start 86 81.405) (end 85.025 81.405) (width 0.5) (layer "F.Cu") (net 2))
 (segment (start 79.85 76) (end 79.35 76.5) (width 0.5) (layer "F.Cu") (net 2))
 (segment (start 83.90001 75.12499) (end 85.53389 75.12499) (width 0.5) (layer "F.Cu") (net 2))
 (segment (start 85.53389 75.12499) (end 86.40001 75.99111) (width 0.5) (layer "F.Cu") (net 2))
 (segment (start 83.5 75.525) (end 83.90001 75.12499) (width 0.5) (layer "F.Cu") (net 2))
 (segment (start 86.40001 75.99111) (end 86.40001 81.00499) (width 0.5) (layer "F.Cu") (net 2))
 (segment (start 85.05 76) (end 85.05 77.57) (width 0.5) (layer "F.Cu") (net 1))
 (segment (start 84.93 77.5) (end 85.025 77.595) (width 0.5) (layer "F.Cu") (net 1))
 (segment (start 85.05 77.57) (end 85.025 77.595) (width 0.5) (layer "F.Cu") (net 1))
 (segment (start 83.5 77.5) (end 84.93 77.5) (width 0.5) (layer "F.Cu") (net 1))
 (via (at 83.5 77.5) (size 0.45) (drill 0.2) (layers "F.Cu" "B.Cu") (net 1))
 (segment (start 84.5 83) (end 84.5 81.5) (width 0.5) (layer "B.Cu") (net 1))
 (segment (start 84 77.5) (end 83.5 77.5) (width 0.5) (layer "B.Cu") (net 1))
 (segment (start 84.5 81.5) (end 85.5 80.5) (width 0.5) (layer "B.Cu") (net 1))
 (segment (start 85.5 80.5) (end 85.5 79) (width 0.5) (layer "B.Cu") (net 1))
 (segment (start 85.5 79) (end 84 77.5) (width 0.5) (layer "B.Cu") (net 1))
 (segment (start 88.59999 81.00499) (end 89 81.405) (width 0.5) (layer "F.Cu") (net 4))
 (segment (start 89.01611 75.12499) (end 88.59999 75.54111) (width 0.5) (layer "F.Cu") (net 4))
 (segment (start 91.05 76) (end 90.17499 75.12499) (width 0.5) (layer "F.Cu") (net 4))
 (segment (start 89 81.405) (end 89.975 81.405) (width 0.5) (layer "F.Cu") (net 4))
 (segment (start 95.65 76.5) (end 91.55 76.5) (width 0.5) (layer "F.Cu") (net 4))
 (segment (start 91.55 76.5) (end 91.05 76) (width 0.5) (layer "F.Cu") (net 4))
 (segment (start 88.59999 75.54111) (end 88.59999 81.00499) (width 0.5) (layer "F.Cu") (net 4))
 (segment (start 90.17499 75.12499) (end 89.01611 75.12499) (width 0.5) (layer "F.Cu") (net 4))
 (segment (start 91.5 77.5) (end 90.07 77.5) (width 0.5) (layer "F.Cu") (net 3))
 (segment (start 89.5 76) (end 89.5 77.12) (width 0.5) (layer "F.Cu") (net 3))
 (segment (start 90.07 77.5) (end 89.975 77.595) (width 0.5) (layer "F.Cu") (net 3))
 (segment (start 89.5 77.12) (end 89.975 77.595) (width 0.5) (layer "F.Cu") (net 3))
 (via (at 91.5 77.5) (size 0.45) (drill 0.2) (layers "F.Cu" "B.Cu") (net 3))
 (segment (start 90.35 83) (end 90.35 81.175) (width 0.5) (layer "B.Cu") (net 3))
 (segment (start 89.175 80) (end 89.175 78.5) (width 0.5) (layer "B.Cu") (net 3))
 (segment (start 90.35 81.175) (end 89.175 80) (width 0.5) (layer "B.Cu") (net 3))
 (segment (start 90.175 77.5) (end 91.5 77.5) (width 0.5) (layer "B.Cu") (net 3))
 (segment (start 89.175 78.5) (end 90.175 77.5) (width 0.5) (layer "B.Cu") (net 3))
 (segment (start 80.965 78.865) (end 80.6 78.5) (width 0.5) (layer "F.Cu") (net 5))
 (segment (start 82.635 78.865) (end 80.965 78.865) (width 0.5) (layer "F.Cu") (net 5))
 (segment (start 85.025 78.865) (end 82.635 78.865) (width 0.5) (layer "F.Cu") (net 5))
 (via (at 82.635 78.865) (size 0.45) (drill 0.2) (layers "F.Cu" "B.Cu") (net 5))
 (segment (start 83.85 79) (end 82.77 79) (width 0.5) (layer "B.Cu") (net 5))
 (segment (start 82.77 79) (end 82.635 78.865) (width 0.5) (layer "B.Cu") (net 5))
 (segment (start 80.965 80.135) (end 80.6 80.5) (width 0.5) (layer "F.Cu") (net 6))
 (segment (start 82.865 80.135) (end 80.965 80.135) (width 0.5) (layer "F.Cu") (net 6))
 (segment (start 85.025 80.135) (end 82.865 80.135) (width 0.5) (layer "F.Cu") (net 6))
 (via (at 82.865 80.135) (size 0.45) (drill 0.2) (layers "F.Cu" "B.Cu") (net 6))
 (segment (start 83.23 80.5) (end 82.865 80.135) (width 0.5) (layer "B.Cu") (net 6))
 (segment (start 83.85 80.5) (end 83.23 80.5) (width 0.5) (layer "B.Cu") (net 6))
 (segment (start 82.85 83) (end 79.9 83) (width 0.5) (layer "B.Cu") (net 10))
 (segment (start 79.9 83) (end 79.4 82.5) (width 0.5) (layer "B.Cu") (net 10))
 (segment (start 94.4 78.5) (end 92 78.5) (width 0.5) (layer "F.Cu") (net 12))
 (segment (start 90.34 78.5) (end 89.975 78.865) (width 0.5) (layer "F.Cu") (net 12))
 (segment (start 92 78.5) (end 90.34 78.5) (width 0.5) (layer "F.Cu") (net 12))
 (via (at 92 78.5) (size 0.45) (drill 0.2) (layers "F.Cu" "B.Cu") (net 12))
 (segment (start 90.825 78.5) (end 92 78.5) (width 0.5) (layer "B.Cu") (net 12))
 (segment (start 92 80.5) (end 90.34 80.5) (width 0.5) (layer "F.Cu") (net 13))
 (segment (start 94.4 80.5) (end 92 80.5) (width 0.5) (layer "F.Cu") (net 13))
 (segment (start 90.34 80.5) (end 89.975 80.135) (width 0.5) (layer "F.Cu") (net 13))
 (via (at 92 80.5) (size 0.45) (drill 0.2) (layers "F.Cu" "B.Cu") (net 13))
 (segment (start 90.825 80) (end 91.5 80) (width 0.5) (layer "B.Cu") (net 13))
 (segment (start 91.5 80) (end 92 80.5) (width 0.5) (layer "B.Cu") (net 13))
 (segment (start 92 83) (end 95.1 83) (width 0.5) (layer "B.Cu") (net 17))
 (segment (start 95.1 83) (end 95.6 82.5) (width 0.5) (layer "B.Cu") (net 17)))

